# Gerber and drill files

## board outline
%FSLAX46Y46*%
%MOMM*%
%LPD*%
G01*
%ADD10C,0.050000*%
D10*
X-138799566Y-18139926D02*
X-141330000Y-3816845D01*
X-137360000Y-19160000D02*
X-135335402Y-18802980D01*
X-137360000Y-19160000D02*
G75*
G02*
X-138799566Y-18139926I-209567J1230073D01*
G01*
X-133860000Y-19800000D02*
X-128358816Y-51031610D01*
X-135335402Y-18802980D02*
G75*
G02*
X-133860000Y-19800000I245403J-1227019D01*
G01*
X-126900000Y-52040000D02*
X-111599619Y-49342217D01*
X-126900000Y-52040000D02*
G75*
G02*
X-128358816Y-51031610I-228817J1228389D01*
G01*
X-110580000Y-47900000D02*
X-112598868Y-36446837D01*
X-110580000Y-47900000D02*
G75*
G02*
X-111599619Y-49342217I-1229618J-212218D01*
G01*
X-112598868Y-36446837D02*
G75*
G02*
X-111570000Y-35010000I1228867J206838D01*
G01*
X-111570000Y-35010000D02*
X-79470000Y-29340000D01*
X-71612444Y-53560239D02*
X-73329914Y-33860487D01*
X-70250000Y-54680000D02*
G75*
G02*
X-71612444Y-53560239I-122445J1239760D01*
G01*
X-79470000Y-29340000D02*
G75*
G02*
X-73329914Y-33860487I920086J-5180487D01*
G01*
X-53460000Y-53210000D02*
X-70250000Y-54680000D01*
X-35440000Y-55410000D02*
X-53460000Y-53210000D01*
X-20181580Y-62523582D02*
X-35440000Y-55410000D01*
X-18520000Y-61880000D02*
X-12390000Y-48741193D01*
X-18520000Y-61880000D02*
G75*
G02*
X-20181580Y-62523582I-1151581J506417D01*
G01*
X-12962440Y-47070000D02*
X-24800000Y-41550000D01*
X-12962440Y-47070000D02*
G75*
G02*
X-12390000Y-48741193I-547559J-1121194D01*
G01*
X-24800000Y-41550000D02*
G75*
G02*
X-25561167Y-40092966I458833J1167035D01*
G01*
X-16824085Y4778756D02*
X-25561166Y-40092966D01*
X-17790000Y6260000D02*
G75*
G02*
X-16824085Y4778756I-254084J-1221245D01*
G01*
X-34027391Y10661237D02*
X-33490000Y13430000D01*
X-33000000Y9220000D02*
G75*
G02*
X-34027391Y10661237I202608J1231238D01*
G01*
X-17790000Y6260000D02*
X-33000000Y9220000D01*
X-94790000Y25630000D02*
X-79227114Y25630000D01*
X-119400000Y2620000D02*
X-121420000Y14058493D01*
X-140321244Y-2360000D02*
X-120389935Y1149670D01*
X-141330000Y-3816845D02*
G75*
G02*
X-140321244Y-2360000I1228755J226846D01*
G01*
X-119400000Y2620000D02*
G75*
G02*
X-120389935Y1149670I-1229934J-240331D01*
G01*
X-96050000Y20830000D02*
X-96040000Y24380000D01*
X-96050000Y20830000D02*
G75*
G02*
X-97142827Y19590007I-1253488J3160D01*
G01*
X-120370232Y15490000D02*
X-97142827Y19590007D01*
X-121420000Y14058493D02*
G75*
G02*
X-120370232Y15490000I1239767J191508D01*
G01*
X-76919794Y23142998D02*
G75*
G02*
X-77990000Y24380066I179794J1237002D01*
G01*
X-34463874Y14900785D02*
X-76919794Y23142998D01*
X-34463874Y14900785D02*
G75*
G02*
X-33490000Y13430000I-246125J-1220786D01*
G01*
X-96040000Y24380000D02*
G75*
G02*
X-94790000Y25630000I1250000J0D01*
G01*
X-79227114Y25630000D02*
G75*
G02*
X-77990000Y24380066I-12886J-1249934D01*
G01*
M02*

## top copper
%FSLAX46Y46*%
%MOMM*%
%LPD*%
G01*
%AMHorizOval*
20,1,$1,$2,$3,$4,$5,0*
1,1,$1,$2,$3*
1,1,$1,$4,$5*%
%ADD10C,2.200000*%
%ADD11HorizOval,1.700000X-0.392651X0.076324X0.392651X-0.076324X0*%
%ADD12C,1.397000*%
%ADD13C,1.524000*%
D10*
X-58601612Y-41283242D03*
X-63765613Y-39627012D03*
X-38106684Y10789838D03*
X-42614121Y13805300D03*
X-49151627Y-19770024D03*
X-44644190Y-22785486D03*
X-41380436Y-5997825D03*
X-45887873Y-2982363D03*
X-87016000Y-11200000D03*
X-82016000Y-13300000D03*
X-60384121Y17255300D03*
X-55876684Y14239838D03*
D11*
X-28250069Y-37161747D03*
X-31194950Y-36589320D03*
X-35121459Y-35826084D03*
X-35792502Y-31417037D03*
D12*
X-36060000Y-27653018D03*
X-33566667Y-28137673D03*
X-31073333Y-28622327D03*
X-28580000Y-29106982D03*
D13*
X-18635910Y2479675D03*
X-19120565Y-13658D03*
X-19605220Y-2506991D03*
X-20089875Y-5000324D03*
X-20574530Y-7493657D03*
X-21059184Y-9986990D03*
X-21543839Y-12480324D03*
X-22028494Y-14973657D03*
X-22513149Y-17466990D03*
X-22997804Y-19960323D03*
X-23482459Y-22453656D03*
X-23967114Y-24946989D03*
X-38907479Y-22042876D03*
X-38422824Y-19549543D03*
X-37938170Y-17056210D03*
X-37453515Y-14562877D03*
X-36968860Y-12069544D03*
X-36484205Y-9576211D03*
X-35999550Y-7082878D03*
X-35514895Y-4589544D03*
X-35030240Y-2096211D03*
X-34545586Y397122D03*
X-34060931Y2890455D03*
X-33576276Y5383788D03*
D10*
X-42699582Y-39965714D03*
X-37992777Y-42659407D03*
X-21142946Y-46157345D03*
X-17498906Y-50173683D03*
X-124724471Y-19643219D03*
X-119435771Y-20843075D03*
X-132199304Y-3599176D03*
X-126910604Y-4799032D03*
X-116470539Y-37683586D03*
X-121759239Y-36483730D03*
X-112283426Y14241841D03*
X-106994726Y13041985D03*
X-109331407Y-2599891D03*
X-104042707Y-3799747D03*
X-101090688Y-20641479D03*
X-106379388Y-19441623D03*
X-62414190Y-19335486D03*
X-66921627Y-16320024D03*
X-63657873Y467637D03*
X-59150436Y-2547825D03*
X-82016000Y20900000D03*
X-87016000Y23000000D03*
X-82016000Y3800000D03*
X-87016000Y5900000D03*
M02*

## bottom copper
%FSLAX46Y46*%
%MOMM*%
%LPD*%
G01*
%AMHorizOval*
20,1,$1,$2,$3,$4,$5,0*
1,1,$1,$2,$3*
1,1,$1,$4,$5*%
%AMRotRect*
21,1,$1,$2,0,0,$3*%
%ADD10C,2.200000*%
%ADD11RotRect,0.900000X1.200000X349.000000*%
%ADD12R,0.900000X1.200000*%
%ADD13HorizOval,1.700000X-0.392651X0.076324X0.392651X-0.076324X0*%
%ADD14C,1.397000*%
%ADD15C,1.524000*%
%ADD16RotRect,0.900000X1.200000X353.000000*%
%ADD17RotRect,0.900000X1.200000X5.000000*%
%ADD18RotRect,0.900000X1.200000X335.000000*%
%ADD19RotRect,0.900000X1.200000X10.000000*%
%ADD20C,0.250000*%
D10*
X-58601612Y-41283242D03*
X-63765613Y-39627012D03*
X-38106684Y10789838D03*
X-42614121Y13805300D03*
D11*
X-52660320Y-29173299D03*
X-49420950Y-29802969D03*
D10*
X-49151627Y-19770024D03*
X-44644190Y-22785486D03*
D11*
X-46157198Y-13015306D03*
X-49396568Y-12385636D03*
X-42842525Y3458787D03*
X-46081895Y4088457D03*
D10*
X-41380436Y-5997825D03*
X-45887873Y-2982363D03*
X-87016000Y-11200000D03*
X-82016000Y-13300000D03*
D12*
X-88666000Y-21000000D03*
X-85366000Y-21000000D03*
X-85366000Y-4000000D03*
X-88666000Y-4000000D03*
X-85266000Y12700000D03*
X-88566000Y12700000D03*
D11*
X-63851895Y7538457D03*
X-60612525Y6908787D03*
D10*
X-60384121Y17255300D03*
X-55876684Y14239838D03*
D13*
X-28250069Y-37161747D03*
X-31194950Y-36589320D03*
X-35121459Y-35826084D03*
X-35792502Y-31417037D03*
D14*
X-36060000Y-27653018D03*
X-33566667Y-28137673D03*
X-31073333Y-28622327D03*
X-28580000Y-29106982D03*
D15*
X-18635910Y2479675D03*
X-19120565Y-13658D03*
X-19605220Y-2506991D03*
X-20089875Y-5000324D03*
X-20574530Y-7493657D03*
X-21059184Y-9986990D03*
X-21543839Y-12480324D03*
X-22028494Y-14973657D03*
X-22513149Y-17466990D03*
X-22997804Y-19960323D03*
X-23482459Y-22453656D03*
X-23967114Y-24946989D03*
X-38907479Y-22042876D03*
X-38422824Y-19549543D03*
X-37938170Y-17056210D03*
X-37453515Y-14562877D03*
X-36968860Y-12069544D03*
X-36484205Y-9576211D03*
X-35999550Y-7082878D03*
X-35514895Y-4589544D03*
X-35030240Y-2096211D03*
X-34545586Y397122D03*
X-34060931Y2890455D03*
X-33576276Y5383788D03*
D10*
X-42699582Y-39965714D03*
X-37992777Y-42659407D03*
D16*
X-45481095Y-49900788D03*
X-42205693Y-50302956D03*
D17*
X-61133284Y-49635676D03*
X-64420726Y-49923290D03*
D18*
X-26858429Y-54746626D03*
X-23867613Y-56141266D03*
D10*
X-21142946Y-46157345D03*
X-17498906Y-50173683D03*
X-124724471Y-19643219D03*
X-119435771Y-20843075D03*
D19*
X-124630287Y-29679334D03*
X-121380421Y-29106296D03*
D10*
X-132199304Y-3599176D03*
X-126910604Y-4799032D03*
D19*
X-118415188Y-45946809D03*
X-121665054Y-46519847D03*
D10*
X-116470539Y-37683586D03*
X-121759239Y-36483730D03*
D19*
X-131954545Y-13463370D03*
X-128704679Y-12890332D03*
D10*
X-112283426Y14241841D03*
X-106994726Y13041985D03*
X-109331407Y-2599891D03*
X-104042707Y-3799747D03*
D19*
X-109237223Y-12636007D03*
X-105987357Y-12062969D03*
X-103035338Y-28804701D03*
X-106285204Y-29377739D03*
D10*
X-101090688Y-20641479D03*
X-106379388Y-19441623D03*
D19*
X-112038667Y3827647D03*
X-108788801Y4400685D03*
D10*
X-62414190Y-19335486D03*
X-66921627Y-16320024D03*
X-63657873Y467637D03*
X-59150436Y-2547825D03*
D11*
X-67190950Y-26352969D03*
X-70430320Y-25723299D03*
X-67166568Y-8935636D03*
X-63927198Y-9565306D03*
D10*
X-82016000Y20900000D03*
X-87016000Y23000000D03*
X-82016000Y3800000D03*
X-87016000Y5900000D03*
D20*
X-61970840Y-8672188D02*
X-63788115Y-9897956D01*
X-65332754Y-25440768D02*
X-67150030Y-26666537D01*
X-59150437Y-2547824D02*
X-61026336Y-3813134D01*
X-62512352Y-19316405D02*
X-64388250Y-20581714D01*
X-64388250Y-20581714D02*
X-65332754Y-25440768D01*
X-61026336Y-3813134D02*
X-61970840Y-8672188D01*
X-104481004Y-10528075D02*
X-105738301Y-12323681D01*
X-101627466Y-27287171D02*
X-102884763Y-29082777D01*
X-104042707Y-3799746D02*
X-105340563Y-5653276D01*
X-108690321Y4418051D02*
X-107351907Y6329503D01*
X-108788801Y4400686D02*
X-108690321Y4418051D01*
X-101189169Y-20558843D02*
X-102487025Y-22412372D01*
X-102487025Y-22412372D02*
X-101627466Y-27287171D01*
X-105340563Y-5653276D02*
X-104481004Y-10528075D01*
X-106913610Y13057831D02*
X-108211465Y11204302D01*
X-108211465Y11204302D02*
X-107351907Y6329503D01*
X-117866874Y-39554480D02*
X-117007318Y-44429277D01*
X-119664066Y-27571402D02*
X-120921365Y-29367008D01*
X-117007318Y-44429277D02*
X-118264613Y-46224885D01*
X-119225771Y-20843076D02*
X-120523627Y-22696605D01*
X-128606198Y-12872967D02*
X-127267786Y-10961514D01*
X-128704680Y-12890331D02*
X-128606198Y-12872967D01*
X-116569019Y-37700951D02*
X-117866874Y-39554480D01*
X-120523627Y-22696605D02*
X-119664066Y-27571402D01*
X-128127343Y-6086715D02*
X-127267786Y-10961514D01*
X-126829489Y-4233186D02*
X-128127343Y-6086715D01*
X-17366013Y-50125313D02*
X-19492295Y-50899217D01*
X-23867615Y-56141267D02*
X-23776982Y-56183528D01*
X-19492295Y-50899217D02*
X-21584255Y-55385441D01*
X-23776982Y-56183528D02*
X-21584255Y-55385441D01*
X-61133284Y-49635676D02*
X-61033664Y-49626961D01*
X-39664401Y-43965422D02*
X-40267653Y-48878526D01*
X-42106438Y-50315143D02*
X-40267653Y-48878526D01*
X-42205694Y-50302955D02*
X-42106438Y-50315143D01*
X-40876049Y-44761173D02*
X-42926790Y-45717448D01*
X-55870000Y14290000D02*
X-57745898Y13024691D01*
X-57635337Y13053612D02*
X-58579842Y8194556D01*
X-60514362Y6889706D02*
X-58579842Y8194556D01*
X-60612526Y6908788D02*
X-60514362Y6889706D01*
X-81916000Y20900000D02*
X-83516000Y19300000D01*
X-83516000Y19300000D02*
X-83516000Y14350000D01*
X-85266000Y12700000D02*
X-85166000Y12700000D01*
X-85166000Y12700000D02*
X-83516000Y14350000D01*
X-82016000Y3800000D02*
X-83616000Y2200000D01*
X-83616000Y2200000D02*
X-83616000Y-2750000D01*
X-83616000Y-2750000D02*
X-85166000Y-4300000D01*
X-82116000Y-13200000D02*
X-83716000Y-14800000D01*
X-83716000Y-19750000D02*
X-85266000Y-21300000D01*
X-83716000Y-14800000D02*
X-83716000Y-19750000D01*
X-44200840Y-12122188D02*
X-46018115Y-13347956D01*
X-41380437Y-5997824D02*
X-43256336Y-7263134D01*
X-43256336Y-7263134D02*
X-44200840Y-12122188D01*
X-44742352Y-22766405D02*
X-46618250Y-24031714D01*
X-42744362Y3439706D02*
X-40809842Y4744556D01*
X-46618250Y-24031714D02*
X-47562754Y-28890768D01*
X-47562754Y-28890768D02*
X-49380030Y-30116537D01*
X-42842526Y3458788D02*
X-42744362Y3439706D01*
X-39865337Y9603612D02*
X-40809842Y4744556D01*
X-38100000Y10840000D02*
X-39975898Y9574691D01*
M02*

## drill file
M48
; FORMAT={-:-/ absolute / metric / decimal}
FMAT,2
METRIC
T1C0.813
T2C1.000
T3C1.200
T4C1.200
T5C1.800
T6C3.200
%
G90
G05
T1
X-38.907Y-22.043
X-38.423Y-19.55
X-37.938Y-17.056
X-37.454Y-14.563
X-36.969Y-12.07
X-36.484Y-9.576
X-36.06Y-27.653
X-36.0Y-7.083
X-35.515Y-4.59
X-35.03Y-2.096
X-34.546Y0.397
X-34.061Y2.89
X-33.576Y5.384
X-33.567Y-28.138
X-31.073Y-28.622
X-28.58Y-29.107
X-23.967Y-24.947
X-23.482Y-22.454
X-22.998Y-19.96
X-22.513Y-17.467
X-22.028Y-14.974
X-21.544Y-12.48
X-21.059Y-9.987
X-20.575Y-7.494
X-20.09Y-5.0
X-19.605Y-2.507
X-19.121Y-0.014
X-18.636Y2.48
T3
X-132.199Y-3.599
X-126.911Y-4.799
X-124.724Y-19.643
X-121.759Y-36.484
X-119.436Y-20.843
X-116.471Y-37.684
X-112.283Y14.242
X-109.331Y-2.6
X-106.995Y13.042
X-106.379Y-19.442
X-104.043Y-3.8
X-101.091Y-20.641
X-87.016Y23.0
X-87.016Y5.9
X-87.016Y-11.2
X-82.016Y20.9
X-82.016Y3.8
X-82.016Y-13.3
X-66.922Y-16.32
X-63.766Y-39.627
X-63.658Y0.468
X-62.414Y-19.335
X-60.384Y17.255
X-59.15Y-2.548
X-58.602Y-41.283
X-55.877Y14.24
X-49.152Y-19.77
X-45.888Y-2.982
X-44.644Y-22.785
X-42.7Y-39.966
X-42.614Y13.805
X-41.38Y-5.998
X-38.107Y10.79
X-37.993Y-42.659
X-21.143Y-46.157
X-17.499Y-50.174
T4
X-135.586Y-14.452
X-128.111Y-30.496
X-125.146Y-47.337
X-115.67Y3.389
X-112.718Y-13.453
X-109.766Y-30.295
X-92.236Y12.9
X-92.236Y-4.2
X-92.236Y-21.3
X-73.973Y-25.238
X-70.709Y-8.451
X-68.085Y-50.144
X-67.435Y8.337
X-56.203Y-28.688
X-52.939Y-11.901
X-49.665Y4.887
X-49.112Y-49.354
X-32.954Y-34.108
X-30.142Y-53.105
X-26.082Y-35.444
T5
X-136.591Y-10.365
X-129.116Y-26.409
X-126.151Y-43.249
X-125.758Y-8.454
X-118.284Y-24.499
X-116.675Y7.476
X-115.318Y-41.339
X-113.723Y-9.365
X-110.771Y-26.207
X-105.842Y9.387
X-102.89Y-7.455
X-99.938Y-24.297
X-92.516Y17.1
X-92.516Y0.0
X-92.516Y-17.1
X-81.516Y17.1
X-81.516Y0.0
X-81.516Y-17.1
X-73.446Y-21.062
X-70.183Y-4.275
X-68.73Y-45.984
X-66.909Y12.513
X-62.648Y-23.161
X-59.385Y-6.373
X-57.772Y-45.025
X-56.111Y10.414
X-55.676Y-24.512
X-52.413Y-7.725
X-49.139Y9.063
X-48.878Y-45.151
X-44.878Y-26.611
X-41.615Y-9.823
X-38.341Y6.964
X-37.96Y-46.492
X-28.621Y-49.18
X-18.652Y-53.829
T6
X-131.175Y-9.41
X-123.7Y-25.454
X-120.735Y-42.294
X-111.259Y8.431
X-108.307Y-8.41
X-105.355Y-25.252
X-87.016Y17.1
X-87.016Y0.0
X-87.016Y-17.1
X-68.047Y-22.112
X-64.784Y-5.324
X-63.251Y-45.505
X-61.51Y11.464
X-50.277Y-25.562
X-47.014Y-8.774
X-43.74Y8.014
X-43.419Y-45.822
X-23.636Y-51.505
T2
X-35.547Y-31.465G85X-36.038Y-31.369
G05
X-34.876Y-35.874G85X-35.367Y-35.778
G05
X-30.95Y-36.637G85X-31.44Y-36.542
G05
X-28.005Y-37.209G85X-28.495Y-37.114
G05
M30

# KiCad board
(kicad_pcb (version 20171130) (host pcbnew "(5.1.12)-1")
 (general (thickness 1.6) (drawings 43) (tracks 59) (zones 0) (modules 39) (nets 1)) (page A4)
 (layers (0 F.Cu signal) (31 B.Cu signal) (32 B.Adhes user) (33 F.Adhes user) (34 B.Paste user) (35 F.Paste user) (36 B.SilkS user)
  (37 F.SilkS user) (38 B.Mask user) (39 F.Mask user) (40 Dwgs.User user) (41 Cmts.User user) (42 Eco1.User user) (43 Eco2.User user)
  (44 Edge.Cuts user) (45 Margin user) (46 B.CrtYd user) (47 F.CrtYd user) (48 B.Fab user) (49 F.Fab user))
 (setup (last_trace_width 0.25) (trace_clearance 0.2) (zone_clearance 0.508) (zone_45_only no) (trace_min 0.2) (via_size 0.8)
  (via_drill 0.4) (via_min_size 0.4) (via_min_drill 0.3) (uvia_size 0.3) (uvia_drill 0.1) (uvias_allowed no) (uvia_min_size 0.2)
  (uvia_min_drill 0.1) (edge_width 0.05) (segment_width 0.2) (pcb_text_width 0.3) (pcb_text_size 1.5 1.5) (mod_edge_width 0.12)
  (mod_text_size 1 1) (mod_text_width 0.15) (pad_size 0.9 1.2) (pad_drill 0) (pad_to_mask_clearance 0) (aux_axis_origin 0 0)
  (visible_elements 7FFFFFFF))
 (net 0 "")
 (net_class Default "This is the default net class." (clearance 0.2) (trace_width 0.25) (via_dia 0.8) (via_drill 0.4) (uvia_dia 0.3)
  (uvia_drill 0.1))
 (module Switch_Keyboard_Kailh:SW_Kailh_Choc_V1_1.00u (layer F.Cu) (at -63.251394 45.504561 5)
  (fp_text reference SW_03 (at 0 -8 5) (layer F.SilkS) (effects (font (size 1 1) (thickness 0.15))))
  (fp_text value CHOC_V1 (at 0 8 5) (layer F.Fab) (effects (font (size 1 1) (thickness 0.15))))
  (pad "" np_thru_hole circle (at -5.22 4.2 5) (size 1.2 1.2) (drill 1.2) (layers *.Cu *.Mask))
  (pad "" np_thru_hole circle (at 5.5 0 5) (size 1.8 1.8) (drill 1.8) (layers *.Cu *.Mask))
  (pad "" np_thru_hole circle (at -5.5 0 5) (size 1.8 1.8) (drill 1.8) (layers *.Cu *.Mask))
  (pad "" np_thru_hole circle (at 0 0 5) (size 3.2 3.2) (drill 3.2) (layers *.Cu *.Mask))
  (pad 2 thru_hole circle (at 5 -3.8 5) (size 2.2 2.2) (drill 1.2) (layers *.Cu B.Mask))
  (pad 1 thru_hole circle (at 0 -5.9 5) (size 2.2 2.2) (drill 1.2) (layers *.Cu B.Mask)))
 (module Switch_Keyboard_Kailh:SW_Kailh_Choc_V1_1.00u (layer F.Cu) (at -43.739894 -8.0137 349)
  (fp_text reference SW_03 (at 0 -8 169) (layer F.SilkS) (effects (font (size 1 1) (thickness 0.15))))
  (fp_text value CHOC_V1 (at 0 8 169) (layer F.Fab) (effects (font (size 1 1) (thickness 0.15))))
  (pad "" np_thru_hole circle (at -5.22 4.2 349) (size 1.2 1.2) (drill 1.2) (layers *.Cu *.Mask))
  (pad "" np_thru_hole circle (at 5.5 0 349) (size 1.8 1.8) (drill 1.8) (layers *.Cu *.Mask))
  (pad "" np_thru_hole circle (at -5.5 0 349) (size 1.8 1.8) (drill 1.8) (layers *.Cu *.Mask))
  (pad "" np_thru_hole circle (at 0 0 349) (size 3.2 3.2) (drill 3.2) (layers *.Cu *.Mask))
  (pad 2 thru_hole circle (at 5 -3.8 349) (size 2.2 2.2) (drill 1.2) (layers *.Cu B.Mask))
  (pad 1 thru_hole circle (at 0 -5.9 349) (size 2.2 2.2) (drill 1.2) (layers *.Cu B.Mask)))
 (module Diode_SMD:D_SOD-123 (layer B.Cu) (at -51.040635 29.488134 349)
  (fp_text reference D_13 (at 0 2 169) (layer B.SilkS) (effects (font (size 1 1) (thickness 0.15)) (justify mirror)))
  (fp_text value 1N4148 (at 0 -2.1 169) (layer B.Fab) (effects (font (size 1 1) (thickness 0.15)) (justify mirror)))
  (pad 1 smd rect (at -1.65 0 349) (size 0.9 1.2) (layers B.Cu B.Paste B.Mask))
  (pad 2 smd rect (at 1.65 0 349) (size 0.9 1.2) (layers B.Cu B.Paste B.Mask)))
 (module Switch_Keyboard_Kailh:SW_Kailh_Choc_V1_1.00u (layer F.Cu) (at -50.2774 25.561624 349)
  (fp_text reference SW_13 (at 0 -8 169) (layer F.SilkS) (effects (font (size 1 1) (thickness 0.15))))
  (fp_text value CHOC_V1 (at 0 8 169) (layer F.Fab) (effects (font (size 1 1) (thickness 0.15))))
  (pad 1 thru_hole circle (at 0 -5.9 349) (size 2.2 2.2) (drill 1.2) (layers *.Cu B.Mask))
  (pad 2 thru_hole circle (at 5 -3.8 349) (size 2.2 2.2) (drill 1.2) (layers *.Cu B.Mask))
  (pad "" np_thru_hole circle (at 0 0 349) (size 3.2 3.2) (drill 3.2) (layers *.Cu *.Mask))
  (pad "" np_thru_hole circle (at -5.5 0 349) (size 1.8 1.8) (drill 1.8) (layers *.Cu *.Mask))
  (pad "" np_thru_hole circle (at 5.5 0 349) (size 1.8 1.8) (drill 1.8) (layers *.Cu *.Mask))
  (pad "" np_thru_hole circle (at -5.22 4.2 349) (size 1.2 1.2) (drill 1.2) (layers *.Cu *.Mask)))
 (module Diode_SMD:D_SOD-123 (layer B.Cu) (at -47.776883 12.700471 349)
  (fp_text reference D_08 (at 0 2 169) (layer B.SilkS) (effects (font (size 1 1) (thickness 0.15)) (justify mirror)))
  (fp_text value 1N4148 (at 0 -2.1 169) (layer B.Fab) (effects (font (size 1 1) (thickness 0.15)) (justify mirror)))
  (pad 2 smd rect (at 1.65 0 349) (size 0.9 1.2) (layers B.Cu B.Paste B.Mask))
  (pad 1 smd rect (at -1.65 0 349) (size 0.9 1.2) (layers B.Cu B.Paste B.Mask)))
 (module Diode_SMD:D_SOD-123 (layer B.Cu) (at -44.46221 -3.773622 349)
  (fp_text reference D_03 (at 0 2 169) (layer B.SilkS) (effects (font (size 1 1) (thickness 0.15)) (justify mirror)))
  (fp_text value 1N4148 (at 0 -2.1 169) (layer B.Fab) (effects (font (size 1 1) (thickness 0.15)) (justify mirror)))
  (pad 2 smd rect (at 1.65 0 349) (size 0.9 1.2) (layers B.Cu B.Paste B.Mask))
  (pad 1 smd rect (at -1.65 0 349) (size 0.9 1.2) (layers B.Cu B.Paste B.Mask)))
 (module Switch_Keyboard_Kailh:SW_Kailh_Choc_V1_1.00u (layer F.Cu) (at -47.013646 8.773963 349)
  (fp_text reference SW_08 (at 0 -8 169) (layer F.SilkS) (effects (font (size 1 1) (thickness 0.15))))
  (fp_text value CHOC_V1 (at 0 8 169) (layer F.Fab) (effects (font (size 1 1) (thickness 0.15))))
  (pad "" np_thru_hole circle (at -5.22 4.2 349) (size 1.2 1.2) (drill 1.2) (layers *.Cu *.Mask))
  (pad "" np_thru_hole circle (at 5.5 0 349) (size 1.8 1.8) (drill 1.8) (layers *.Cu *.Mask))
  (pad "" np_thru_hole circle (at -5.5 0 349) (size 1.8 1.8) (drill 1.8) (layers *.Cu *.Mask))
  (pad "" np_thru_hole circle (at 0 0 349) (size 3.2 3.2) (drill 3.2) (layers *.Cu *.Mask))
  (pad 2 thru_hole circle (at 5 -3.8 349) (size 2.2 2.2) (drill 1.2) (layers *.Cu B.Mask))
  (pad 1 thru_hole circle (at 0 -5.9 349) (size 2.2 2.2) (drill 1.2) (layers *.Cu B.Mask)))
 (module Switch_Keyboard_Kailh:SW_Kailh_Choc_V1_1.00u (layer F.Cu) (at -87.016 17.1)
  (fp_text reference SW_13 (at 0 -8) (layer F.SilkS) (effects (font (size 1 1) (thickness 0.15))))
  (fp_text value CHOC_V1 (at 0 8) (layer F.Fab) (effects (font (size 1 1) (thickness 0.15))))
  (pad 1 thru_hole circle (at 0 -5.9) (size 2.2 2.2) (drill 1.2) (layers *.Cu B.Mask))
  (pad 2 thru_hole circle (at 5 -3.8) (size 2.2 2.2) (drill 1.2) (layers *.Cu B.Mask))
  (pad "" np_thru_hole circle (at 0 0) (size 3.2 3.2) (drill 3.2) (layers *.Cu *.Mask))
  (pad "" np_thru_hole circle (at -5.5 0) (size 1.8 1.8) (drill 1.8) (layers *.Cu *.Mask))
  (pad "" np_thru_hole circle (at 5.5 0) (size 1.8 1.8) (drill 1.8) (layers *.Cu *.Mask))
  (pad "" np_thru_hole circle (at -5.22 4.2) (size 1.2 1.2) (drill 1.2) (layers *.Cu *.Mask)))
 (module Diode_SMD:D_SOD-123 (layer B.Cu) (at -87.016 21)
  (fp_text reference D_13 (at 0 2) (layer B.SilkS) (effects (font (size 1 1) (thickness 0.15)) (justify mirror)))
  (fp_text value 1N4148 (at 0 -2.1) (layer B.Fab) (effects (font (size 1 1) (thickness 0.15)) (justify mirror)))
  (pad 1 smd rect (at -1.65 0) (size 0.9 1.2) (layers B.Cu B.Paste B.Mask))
  (pad 2 smd rect (at 1.65 0) (size 0.9 1.2) (layers B.Cu B.Paste B.Mask)))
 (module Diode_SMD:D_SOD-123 (layer B.Cu) (at -87.016 4)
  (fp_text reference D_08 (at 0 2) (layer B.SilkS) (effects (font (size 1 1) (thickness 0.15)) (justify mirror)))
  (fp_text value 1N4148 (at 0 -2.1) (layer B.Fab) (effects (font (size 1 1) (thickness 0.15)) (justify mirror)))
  (pad 2 smd rect (at 1.65 0) (size 0.9 1.2) (layers B.Cu B.Paste B.Mask))
  (pad 1 smd rect (at -1.65 0) (size 0.9 1.2) (layers B.Cu B.Paste B.Mask)))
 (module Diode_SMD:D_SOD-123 (layer B.Cu) (at -86.916 -12.7)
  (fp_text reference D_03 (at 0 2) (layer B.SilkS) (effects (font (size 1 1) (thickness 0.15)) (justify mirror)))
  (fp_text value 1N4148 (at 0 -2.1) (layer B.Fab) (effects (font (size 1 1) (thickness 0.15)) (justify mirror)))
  (pad 2 smd rect (at 1.65 0) (size 0.9 1.2) (layers B.Cu B.Paste B.Mask))
  (pad 1 smd rect (at -1.65 0) (size 0.9 1.2) (layers B.Cu B.Paste B.Mask)))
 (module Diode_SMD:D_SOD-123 (layer B.Cu) (at -62.23221 -7.223622 349)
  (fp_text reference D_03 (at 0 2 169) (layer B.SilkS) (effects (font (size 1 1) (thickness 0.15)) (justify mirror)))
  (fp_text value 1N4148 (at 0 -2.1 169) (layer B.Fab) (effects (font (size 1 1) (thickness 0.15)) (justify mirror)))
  (pad 1 smd rect (at -1.65 0 349) (size 0.9 1.2) (layers B.Cu B.Paste B.Mask))
  (pad 2 smd rect (at 1.65 0 349) (size 0.9 1.2) (layers B.Cu B.Paste B.Mask)))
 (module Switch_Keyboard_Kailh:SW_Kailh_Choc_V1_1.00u (layer F.Cu) (at -61.509894 -11.4637 349)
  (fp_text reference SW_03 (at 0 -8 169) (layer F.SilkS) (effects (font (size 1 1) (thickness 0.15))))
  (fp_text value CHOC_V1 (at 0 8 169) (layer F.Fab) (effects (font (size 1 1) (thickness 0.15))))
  (pad 1 thru_hole circle (at 0 -5.9 349) (size 2.2 2.2) (drill 1.2) (layers *.Cu B.Mask))
  (pad 2 thru_hole circle (at 5 -3.8 349) (size 2.2 2.2) (drill 1.2) (layers *.Cu B.Mask))
  (pad "" np_thru_hole circle (at 0 0 349) (size 3.2 3.2) (drill 3.2) (layers *.Cu *.Mask))
  (pad "" np_thru_hole circle (at -5.5 0 349) (size 1.8 1.8) (drill 1.8) (layers *.Cu *.Mask))
  (pad "" np_thru_hole circle (at 5.5 0 349) (size 1.8 1.8) (drill 1.8) (layers *.Cu *.Mask))
  (pad "" np_thru_hole circle (at -5.22 4.2 349) (size 1.2 1.2) (drill 1.2) (layers *.Cu *.Mask)))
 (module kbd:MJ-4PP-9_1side (layer F.Cu) (at -24.61 35.73 259)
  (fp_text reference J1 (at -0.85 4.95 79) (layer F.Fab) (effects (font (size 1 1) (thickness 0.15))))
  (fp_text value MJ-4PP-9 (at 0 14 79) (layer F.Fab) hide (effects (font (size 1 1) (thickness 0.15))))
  (pad "" np_thru_hole circle (at 0 1.5 259) (size 1.2 1.2) (drill 1.2) (layers *.Cu *.Mask))
  (pad "" np_thru_hole circle (at 0 8.5 259) (size 1.2 1.2) (drill 1.2) (layers *.Cu *.Mask))
  (pad B thru_hole oval (at 2.1 3.3 259) (size 1.7 2.5) (drill oval 1 1.5) (layers *.Cu B.Mask))
  (pad C thru_hole oval (at 2.1 6.3 259) (size 1.7 2.5) (drill oval 1 1.5) (layers *.Cu B.Mask))
  (pad D thru_hole oval (at 2.1 10.3 259) (size 1.7 2.5) (drill oval 1 1.5) (layers *.Cu B.Mask) (clearance 0.15))
  (pad A thru_hole oval (at -2.1 11.8 259) (size 1.7 2.5) (drill oval 1 1.5) (layers *.Cu B.Mask) (clearance 0.15)))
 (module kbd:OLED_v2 (layer F.Cu) (at -32.32 28.38 349)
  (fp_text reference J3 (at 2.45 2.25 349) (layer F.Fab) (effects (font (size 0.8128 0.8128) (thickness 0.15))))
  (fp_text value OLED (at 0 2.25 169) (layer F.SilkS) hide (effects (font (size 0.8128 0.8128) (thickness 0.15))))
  (pad 1 thru_hole circle (at -3.81 0 349) (size 1.397 1.397) (drill 0.8128) (layers *.Cu F.SilkS B.Mask))
  (pad 2 thru_hole circle (at -1.27 0 349) (size 1.397 1.397) (drill 0.8128) (layers *.Cu F.SilkS B.Mask))
  (pad 3 thru_hole circle (at 1.27 0 349) (size 1.397 1.397) (drill 0.8128) (layers *.Cu F.SilkS B.Mask))
  (pad 4 thru_hole circle (at 3.81 0 349) (size 1.397 1.397) (drill 0.8128) (layers *.Cu F.SilkS B.Mask)))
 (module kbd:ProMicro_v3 (layer F.Cu) (at -28.87 10.28 349)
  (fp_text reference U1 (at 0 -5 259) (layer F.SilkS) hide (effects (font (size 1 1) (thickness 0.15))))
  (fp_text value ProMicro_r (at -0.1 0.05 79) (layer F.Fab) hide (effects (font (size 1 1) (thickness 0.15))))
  (pad 1 thru_hole circle (at 7.6114 -14.478 349) (size 1.524 1.524) (drill 0.8128) (layers *.Cu B.Mask))
  (pad 2 thru_hole circle (at 7.6114 -11.938 349) (size 1.524 1.524) (drill 0.8128) (layers *.Cu B.Mask))
  (pad 3 thru_hole circle (at 7.6114 -9.398 349) (size 1.524 1.524) (drill 0.8128) (layers *.Cu B.Mask))
  (pad 4 thru_hole circle (at 7.6114 -6.858 349) (size 1.524 1.524) (drill 0.8128) (layers *.Cu B.Mask))
  (pad 5 thru_hole circle (at 7.6114 -4.318 349) (size 1.524 1.524) (drill 0.8128) (layers *.Cu B.Mask))
  (pad 6 thru_hole circle (at 7.6114 -1.778 349) (size 1.524 1.524) (drill 0.8128) (layers *.Cu B.Mask))
  (pad 7 thru_hole circle (at 7.6114 0.762 349) (size 1.524 1.524) (drill 0.8128) (layers *.Cu B.Mask))
  (pad 8 thru_hole circle (at 7.6114 3.302 349) (size 1.524 1.524) (drill 0.8128) (layers *.Cu B.Mask))
  (pad 9 thru_hole circle (at 7.6114 5.842 349) (size 1.524 1.524) (drill 0.8128) (layers *.Cu B.Mask))
  (pad 10 thru_hole circle (at 7.6114 8.382 349) (size 1.524 1.524) (drill 0.8128) (layers *.Cu B.Mask))
  (pad 11 thru_hole circle (at 7.6114 10.922 349) (size 1.524 1.524) (drill 0.8128) (layers *.Cu B.Mask))
  (pad 12 thru_hole circle (at 7.6114 13.462 349) (size 1.524 1.524) (drill 0.8128) (layers *.Cu B.Mask))
  (pad 13 thru_hole circle (at -7.6086 13.462 349) (size 1.524 1.524) (drill 0.8128) (layers *.Cu B.Mask))
  (pad 14 thru_hole circle (at -7.6086 10.922 349) (size 1.524 1.524) (drill 0.8128) (layers *.Cu B.Mask))
  (pad 15 thru_hole circle (at -7.6086 8.382 349) (size 1.524 1.524) (drill 0.8128) (layers *.Cu B.Mask))
  (pad 16 thru_hole circle (at -7.6086 5.842 349) (size 1.524 1.524) (drill 0.8128) (layers *.Cu B.Mask))
  (pad 17 thru_hole circle (at -7.6086 3.302 349) (size 1.524 1.524) (drill 0.8128) (layers *.Cu B.Mask))
  (pad 18 thru_hole circle (at -7.6086 0.762 349) (size 1.524 1.524) (drill 0.8128) (layers *.Cu B.Mask))
  (pad 19 thru_hole circle (at -7.6086 -1.778 349) (size 1.524 1.524) (drill 0.8128) (layers *.Cu B.Mask))
  (pad 20 thru_hole circle (at -7.6086 -4.318 349) (size 1.524 1.524) (drill 0.8128) (layers *.Cu B.Mask))
  (pad 21 thru_hole circle (at -7.6086 -6.858 349) (size 1.524 1.524) (drill 0.8128) (layers *.Cu B.Mask))
  (pad 22 thru_hole circle (at -7.6086 -9.398 349) (size 1.524 1.524) (drill 0.8128) (layers *.Cu B.Mask))
  (pad 23 thru_hole circle (at -7.6086 -11.938 349) (size 1.524 1.524) (drill 0.8128) (layers *.Cu B.Mask))
  (pad 24 thru_hole circle (at -7.6086 -14.478 349) (size 1.524 1.524) (drill 0.8128) (layers *.Cu B.Mask)))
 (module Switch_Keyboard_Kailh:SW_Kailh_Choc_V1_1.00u (layer F.Cu) (at -43.418611 45.821736 353)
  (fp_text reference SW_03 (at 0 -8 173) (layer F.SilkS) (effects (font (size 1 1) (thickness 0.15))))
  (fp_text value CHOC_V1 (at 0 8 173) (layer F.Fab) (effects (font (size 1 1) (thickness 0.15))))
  (pad 1 thru_hole circle (at 0 -5.9 353) (size 2.2 2.2) (drill 1.2) (layers *.Cu B.Mask))
  (pad 2 thru_hole circle (at 5 -3.8 353) (size 2.2 2.2) (drill 1.2) (layers *.Cu B.Mask))
  (pad "" np_thru_hole circle (at 0 0 353) (size 3.2 3.2) (drill 3.2) (layers *.Cu *.Mask))
  (pad "" np_thru_hole circle (at -5.5 0 353) (size 1.8 1.8) (drill 1.8) (layers *.Cu *.Mask))
  (pad "" np_thru_hole circle (at 5.5 0 353) (size 1.8 1.8) (drill 1.8) (layers *.Cu *.Mask))
  (pad "" np_thru_hole circle (at -5.22 4.2 353) (size 1.2 1.2) (drill 1.2) (layers *.Cu *.Mask)))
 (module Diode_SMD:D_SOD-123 (layer B.Cu) (at -43.843394 50.101872 353)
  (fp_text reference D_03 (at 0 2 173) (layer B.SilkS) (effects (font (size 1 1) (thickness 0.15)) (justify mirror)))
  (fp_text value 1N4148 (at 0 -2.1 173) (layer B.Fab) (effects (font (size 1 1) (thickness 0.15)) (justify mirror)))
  (pad 1 smd rect (at -1.65 0 353) (size 0.9 1.2) (layers B.Cu B.Paste B.Mask))
  (pad 2 smd rect (at 1.65 0 353) (size 0.9 1.2) (layers B.Cu B.Paste B.Mask)))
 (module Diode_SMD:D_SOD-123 (layer B.Cu) (at -62.777005 49.779483 5)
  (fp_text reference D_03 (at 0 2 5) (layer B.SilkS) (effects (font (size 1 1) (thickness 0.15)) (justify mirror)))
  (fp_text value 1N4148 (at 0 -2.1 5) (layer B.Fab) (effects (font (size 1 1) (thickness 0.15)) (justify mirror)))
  (pad 2 smd rect (at 1.65 0 5) (size 0.9 1.2) (layers B.Cu B.Paste B.Mask))
  (pad 1 smd rect (at -1.65 0 5) (size 0.9 1.2) (layers B.Cu B.Paste B.Mask)))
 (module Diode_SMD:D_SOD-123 (layer B.Cu) (at -25.363021 55.443946 335)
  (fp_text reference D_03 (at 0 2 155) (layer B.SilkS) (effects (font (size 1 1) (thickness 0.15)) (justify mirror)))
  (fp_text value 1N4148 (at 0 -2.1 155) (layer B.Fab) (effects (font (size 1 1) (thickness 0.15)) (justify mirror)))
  (pad 1 smd rect (at -1.65 0 335) (size 0.9 1.2) (layers B.Cu B.Paste B.Mask))
  (pad 2 smd rect (at 1.65 0 335) (size 0.9 1.2) (layers B.Cu B.Paste B.Mask)))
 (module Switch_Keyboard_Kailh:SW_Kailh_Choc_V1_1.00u (layer F.Cu) (at -23.636394 51.504561 335)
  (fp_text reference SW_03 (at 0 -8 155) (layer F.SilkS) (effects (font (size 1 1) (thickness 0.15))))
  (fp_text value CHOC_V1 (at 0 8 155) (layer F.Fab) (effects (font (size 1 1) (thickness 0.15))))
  (pad 1 thru_hole circle (at 0 -5.9 335) (size 2.2 2.2) (drill 1.2) (layers *.Cu B.Mask))
  (pad 2 thru_hole circle (at 5 -3.8 335) (size 2.2 2.2) (drill 1.2) (layers *.Cu B.Mask))
  (pad "" np_thru_hole circle (at 0 0 335) (size 3.2 3.2) (drill 3.2) (layers *.Cu *.Mask))
  (pad "" np_thru_hole circle (at -5.5 0 335) (size 1.8 1.8) (drill 1.8) (layers *.Cu *.Mask))
  (pad "" np_thru_hole circle (at 5.5 0 335) (size 1.8 1.8) (drill 1.8) (layers *.Cu *.Mask))
  (pad "" np_thru_hole circle (at -5.22 4.2 335) (size 1.2 1.2) (drill 1.2) (layers *.Cu *.Mask)))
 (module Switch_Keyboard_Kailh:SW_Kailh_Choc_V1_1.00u (layer F.Cu) (at -123.699947 25.453585 10)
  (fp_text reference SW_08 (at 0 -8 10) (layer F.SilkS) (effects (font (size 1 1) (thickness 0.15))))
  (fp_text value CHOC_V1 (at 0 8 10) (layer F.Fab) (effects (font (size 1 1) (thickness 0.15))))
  (pad 1 thru_hole circle (at 0 -5.9 10) (size 2.2 2.2) (drill 1.2) (layers *.Cu B.Mask))
  (pad 2 thru_hole circle (at 5 -3.8 10) (size 2.2 2.2) (drill 1.2) (layers *.Cu B.Mask))
  (pad "" np_thru_hole circle (at 0 0 10) (size 3.2 3.2) (drill 3.2) (layers *.Cu *.Mask))
  (pad "" np_thru_hole circle (at -5.5 0 10) (size 1.8 1.8) (drill 1.8) (layers *.Cu *.Mask))
  (pad "" np_thru_hole circle (at 5.5 0 10) (size 1.8 1.8) (drill 1.8) (layers *.Cu *.Mask))
  (pad "" np_thru_hole circle (at -5.22 4.2 10) (size 1.2 1.2) (drill 1.2) (layers *.Cu *.Mask)))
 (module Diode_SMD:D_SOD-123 (layer B.Cu) (at -123.005354 29.392815 10)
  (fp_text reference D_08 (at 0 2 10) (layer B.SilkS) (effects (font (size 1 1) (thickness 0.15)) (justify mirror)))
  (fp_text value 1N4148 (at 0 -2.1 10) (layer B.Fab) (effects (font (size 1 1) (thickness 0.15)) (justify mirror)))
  (pad 1 smd rect (at -1.65 0 10) (size 0.9 1.2) (layers B.Cu B.Paste B.Mask))
  (pad 2 smd rect (at 1.65 0 10) (size 0.9 1.2) (layers B.Cu B.Paste B.Mask)))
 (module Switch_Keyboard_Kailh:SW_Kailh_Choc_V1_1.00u (layer F.Cu) (at -131.17478 9.409542 10)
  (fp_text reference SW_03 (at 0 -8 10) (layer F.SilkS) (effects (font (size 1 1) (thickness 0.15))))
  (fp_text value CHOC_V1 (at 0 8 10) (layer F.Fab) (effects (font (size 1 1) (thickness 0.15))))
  (pad 1 thru_hole circle (at 0 -5.9 10) (size 2.2 2.2) (drill 1.2) (layers *.Cu B.Mask))
  (pad 2 thru_hole circle (at 5 -3.8 10) (size 2.2 2.2) (drill 1.2) (layers *.Cu B.Mask))
  (pad "" np_thru_hole circle (at 0 0 10) (size 3.2 3.2) (drill 3.2) (layers *.Cu *.Mask))
  (pad "" np_thru_hole circle (at -5.5 0 10) (size 1.8 1.8) (drill 1.8) (layers *.Cu *.Mask))
  (pad "" np_thru_hole circle (at 5.5 0 10) (size 1.8 1.8) (drill 1.8) (layers *.Cu *.Mask))
  (pad "" np_thru_hole circle (at -5.22 4.2 10) (size 1.2 1.2) (drill 1.2) (layers *.Cu *.Mask)))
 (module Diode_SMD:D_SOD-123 (layer B.Cu) (at -120.040121 46.233328 10)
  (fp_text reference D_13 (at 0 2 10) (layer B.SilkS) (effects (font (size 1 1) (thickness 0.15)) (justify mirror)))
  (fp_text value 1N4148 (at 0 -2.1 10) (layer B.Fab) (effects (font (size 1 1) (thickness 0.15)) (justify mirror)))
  (pad 2 smd rect (at 1.65 0 10) (size 0.9 1.2) (layers B.Cu B.Paste B.Mask))
  (pad 1 smd rect (at -1.65 0 10) (size 0.9 1.2) (layers B.Cu B.Paste B.Mask)))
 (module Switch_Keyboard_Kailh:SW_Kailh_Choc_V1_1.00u (layer F.Cu) (at -120.734715 42.294096 10)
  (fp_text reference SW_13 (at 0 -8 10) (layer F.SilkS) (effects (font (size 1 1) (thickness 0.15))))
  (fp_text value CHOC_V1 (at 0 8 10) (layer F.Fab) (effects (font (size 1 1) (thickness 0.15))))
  (pad "" np_thru_hole circle (at -5.22 4.2 10) (size 1.2 1.2) (drill 1.2) (layers *.Cu *.Mask))
  (pad "" np_thru_hole circle (at 5.5 0 10) (size 1.8 1.8) (drill 1.8) (layers *.Cu *.Mask))
  (pad "" np_thru_hole circle (at -5.5 0 10) (size 1.8 1.8) (drill 1.8) (layers *.Cu *.Mask))
  (pad "" np_thru_hole circle (at 0 0 10) (size 3.2 3.2) (drill 3.2) (layers *.Cu *.Mask))
  (pad 2 thru_hole circle (at 5 -3.8 10) (size 2.2 2.2) (drill 1.2) (layers *.Cu B.Mask))
  (pad 1 thru_hole circle (at 0 -5.9 10) (size 2.2 2.2) (drill 1.2) (layers *.Cu B.Mask)))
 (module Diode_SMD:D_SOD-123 (layer B.Cu) (at -130.329612 13.176851 10)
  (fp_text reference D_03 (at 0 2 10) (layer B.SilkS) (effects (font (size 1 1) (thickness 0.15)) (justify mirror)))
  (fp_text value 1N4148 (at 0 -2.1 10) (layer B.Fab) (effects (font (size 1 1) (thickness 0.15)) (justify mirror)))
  (pad 1 smd rect (at -1.65 0 10) (size 0.9 1.2) (layers B.Cu B.Paste B.Mask))
  (pad 2 smd rect (at 1.65 0 10) (size 0.9 1.2) (layers B.Cu B.Paste B.Mask)))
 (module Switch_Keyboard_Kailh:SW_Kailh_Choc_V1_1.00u (layer F.Cu) (at -111.258902 -8.431475 10)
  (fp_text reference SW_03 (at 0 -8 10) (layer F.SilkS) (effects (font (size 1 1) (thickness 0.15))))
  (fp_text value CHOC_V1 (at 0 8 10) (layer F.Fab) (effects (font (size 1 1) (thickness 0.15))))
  (pad 1 thru_hole circle (at 0 -5.9 10) (size 2.2 2.2) (drill 1.2) (layers *.Cu B.Mask))
  (pad 2 thru_hole circle (at 5 -3.8 10) (size 2.2 2.2) (drill 1.2) (layers *.Cu B.Mask))
  (pad "" np_thru_hole circle (at 0 0 10) (size 3.2 3.2) (drill 3.2) (layers *.Cu *.Mask))
  (pad "" np_thru_hole circle (at -5.5 0 10) (size 1.8 1.8) (drill 1.8) (layers *.Cu *.Mask))
  (pad "" np_thru_hole circle (at 5.5 0 10) (size 1.8 1.8) (drill 1.8) (layers *.Cu *.Mask))
  (pad "" np_thru_hole circle (at -5.22 4.2 10) (size 1.2 1.2) (drill 1.2) (layers *.Cu *.Mask)))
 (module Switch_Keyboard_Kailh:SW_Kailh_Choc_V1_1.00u (layer F.Cu) (at -108.306883 8.410257 10)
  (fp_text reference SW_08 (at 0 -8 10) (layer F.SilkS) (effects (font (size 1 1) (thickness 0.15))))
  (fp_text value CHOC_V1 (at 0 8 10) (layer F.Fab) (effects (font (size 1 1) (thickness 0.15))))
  (pad 1 thru_hole circle (at 0 -5.9 10) (size 2.2 2.2) (drill 1.2) (layers *.Cu B.Mask))
  (pad 2 thru_hole circle (at 5 -3.8 10) (size 2.2 2.2) (drill 1.2) (layers *.Cu B.Mask))
  (pad "" np_thru_hole circle (at 0 0 10) (size 3.2 3.2) (drill 3.2) (layers *.Cu *.Mask))
  (pad "" np_thru_hole circle (at -5.5 0 10) (size 1.8 1.8) (drill 1.8) (layers *.Cu *.Mask))
  (pad "" np_thru_hole circle (at 5.5 0 10) (size 1.8 1.8) (drill 1.8) (layers *.Cu *.Mask))
  (pad "" np_thru_hole circle (at -5.22 4.2 10) (size 1.2 1.2) (drill 1.2) (layers *.Cu *.Mask)))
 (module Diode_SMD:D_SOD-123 (layer B.Cu) (at -107.61229 12.349488 10)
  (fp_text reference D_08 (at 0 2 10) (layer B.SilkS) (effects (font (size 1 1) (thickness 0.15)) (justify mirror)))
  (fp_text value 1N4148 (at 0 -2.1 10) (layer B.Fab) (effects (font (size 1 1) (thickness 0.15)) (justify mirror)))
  (pad 1 smd rect (at -1.65 0 10) (size 0.9 1.2) (layers B.Cu B.Paste B.Mask))
  (pad 2 smd rect (at 1.65 0 10) (size 0.9 1.2) (layers B.Cu B.Paste B.Mask)))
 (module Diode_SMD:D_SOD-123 (layer B.Cu) (at -104.660271 29.09122 10)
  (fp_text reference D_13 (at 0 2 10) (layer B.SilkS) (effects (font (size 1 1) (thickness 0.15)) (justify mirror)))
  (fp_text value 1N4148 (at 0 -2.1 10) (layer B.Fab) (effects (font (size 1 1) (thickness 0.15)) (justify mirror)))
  (pad 2 smd rect (at 1.65 0 10) (size 0.9 1.2) (layers B.Cu B.Paste B.Mask))
  (pad 1 smd rect (at -1.65 0 10) (size 0.9 1.2) (layers B.Cu B.Paste B.Mask)))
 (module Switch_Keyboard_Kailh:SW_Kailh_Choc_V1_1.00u (layer F.Cu) (at -105.354864 25.251989 10)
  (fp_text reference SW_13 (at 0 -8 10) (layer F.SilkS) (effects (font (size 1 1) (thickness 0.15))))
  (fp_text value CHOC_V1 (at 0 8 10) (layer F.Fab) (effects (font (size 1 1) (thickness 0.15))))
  (pad "" np_thru_hole circle (at -5.22 4.2 10) (size 1.2 1.2) (drill 1.2) (layers *.Cu *.Mask))
  (pad "" np_thru_hole circle (at 5.5 0 10) (size 1.8 1.8) (drill 1.8) (layers *.Cu *.Mask))
  (pad "" np_thru_hole circle (at -5.5 0 10) (size 1.8 1.8) (drill 1.8) (layers *.Cu *.Mask))
  (pad "" np_thru_hole circle (at 0 0 10) (size 3.2 3.2) (drill 3.2) (layers *.Cu *.Mask))
  (pad 2 thru_hole circle (at 5 -3.8 10) (size 2.2 2.2) (drill 1.2) (layers *.Cu B.Mask))
  (pad 1 thru_hole circle (at 0 -5.9 10) (size 2.2 2.2) (drill 1.2) (layers *.Cu B.Mask)))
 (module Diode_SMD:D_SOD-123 (layer B.Cu) (at -110.413734 -4.114166 10)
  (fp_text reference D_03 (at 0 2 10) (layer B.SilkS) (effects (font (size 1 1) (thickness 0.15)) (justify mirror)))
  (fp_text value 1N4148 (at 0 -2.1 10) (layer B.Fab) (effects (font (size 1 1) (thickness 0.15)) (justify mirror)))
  (pad 1 smd rect (at -1.65 0 10) (size 0.9 1.2) (layers B.Cu B.Paste B.Mask))
  (pad 2 smd rect (at 1.65 0 10) (size 0.9 1.2) (layers B.Cu B.Paste B.Mask)))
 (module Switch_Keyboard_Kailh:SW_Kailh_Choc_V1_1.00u (layer F.Cu) (at -68.0474 22.111624 349)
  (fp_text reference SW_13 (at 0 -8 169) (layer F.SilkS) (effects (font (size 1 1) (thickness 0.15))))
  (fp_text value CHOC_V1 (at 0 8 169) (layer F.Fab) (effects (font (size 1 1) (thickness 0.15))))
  (pad "" np_thru_hole circle (at -5.22 4.2 349) (size 1.2 1.2) (drill 1.2) (layers *.Cu *.Mask))
  (pad "" np_thru_hole circle (at 5.5 0 349) (size 1.8 1.8) (drill 1.8) (layers *.Cu *.Mask))
  (pad "" np_thru_hole circle (at -5.5 0 349) (size 1.8 1.8) (drill 1.8) (layers *.Cu *.Mask))
  (pad "" np_thru_hole circle (at 0 0 349) (size 3.2 3.2) (drill 3.2) (layers *.Cu *.Mask))
  (pad 2 thru_hole circle (at 5 -3.8 349) (size 2.2 2.2) (drill 1.2) (layers *.Cu B.Mask))
  (pad 1 thru_hole circle (at 0 -5.9 349) (size 2.2 2.2) (drill 1.2) (layers *.Cu B.Mask)))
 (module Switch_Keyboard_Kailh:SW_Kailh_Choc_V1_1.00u (layer F.Cu) (at -64.783646 5.323963 349)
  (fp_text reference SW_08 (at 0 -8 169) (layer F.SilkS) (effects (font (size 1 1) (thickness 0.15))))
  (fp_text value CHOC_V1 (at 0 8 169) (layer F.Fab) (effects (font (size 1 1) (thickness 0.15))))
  (pad 1 thru_hole circle (at 0 -5.9 349) (size 2.2 2.2) (drill 1.2) (layers *.Cu B.Mask))
  (pad 2 thru_hole circle (at 5 -3.8 349) (size 2.2 2.2) (drill 1.2) (layers *.Cu B.Mask))
  (pad "" np_thru_hole circle (at 0 0 349) (size 3.2 3.2) (drill 3.2) (layers *.Cu *.Mask))
  (pad "" np_thru_hole circle (at -5.5 0 349) (size 1.8 1.8) (drill 1.8) (layers *.Cu *.Mask))
  (pad "" np_thru_hole circle (at 5.5 0 349) (size 1.8 1.8) (drill 1.8) (layers *.Cu *.Mask))
  (pad "" np_thru_hole circle (at -5.22 4.2 349) (size 1.2 1.2) (drill 1.2) (layers *.Cu *.Mask)))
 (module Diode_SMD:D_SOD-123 (layer B.Cu) (at -68.810635 26.038134 349)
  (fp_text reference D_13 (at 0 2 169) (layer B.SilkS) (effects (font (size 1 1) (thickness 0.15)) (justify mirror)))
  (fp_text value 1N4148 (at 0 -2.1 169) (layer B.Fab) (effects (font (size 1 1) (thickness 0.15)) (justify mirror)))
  (pad 2 smd rect (at 1.65 0 349) (size 0.9 1.2) (layers B.Cu B.Paste B.Mask))
  (pad 1 smd rect (at -1.65 0 349) (size 0.9 1.2) (layers B.Cu B.Paste B.Mask)))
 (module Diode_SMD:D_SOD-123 (layer B.Cu) (at -65.546883 9.250471 349)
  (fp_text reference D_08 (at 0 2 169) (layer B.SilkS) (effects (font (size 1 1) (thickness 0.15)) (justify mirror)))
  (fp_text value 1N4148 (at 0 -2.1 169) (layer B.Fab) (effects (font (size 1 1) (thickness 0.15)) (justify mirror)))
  (pad 1 smd rect (at -1.65 0 349) (size 0.9 1.2) (layers B.Cu B.Paste B.Mask))
  (pad 2 smd rect (at 1.65 0 349) (size 0.9 1.2) (layers B.Cu B.Paste B.Mask)))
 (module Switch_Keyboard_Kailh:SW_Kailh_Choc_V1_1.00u (layer F.Cu) (at -87.016 -17.1)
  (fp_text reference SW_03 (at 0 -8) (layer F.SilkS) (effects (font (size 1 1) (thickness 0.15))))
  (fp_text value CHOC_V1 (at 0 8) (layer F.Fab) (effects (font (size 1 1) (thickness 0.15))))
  (pad "" np_thru_hole circle (at -5.22 4.2) (size 1.2 1.2) (drill 1.2) (layers *.Cu *.Mask))
  (pad "" np_thru_hole circle (at 5.5 0) (size 1.8 1.8) (drill 1.8) (layers *.Cu *.Mask))
  (pad "" np_thru_hole circle (at -5.5 0) (size 1.8 1.8) (drill 1.8) (layers *.Cu *.Mask))
  (pad "" np_thru_hole circle (at 0 0) (size 3.2 3.2) (drill 3.2) (layers *.Cu *.Mask))
  (pad 2 thru_hole circle (at 5 -3.8) (size 2.2 2.2) (drill 1.2) (layers *.Cu B.Mask))
  (pad 1 thru_hole circle (at 0 -5.9) (size 2.2 2.2) (drill 1.2) (layers *.Cu B.Mask)))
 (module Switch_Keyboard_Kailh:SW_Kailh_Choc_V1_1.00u (layer F.Cu) (at -87.016 0)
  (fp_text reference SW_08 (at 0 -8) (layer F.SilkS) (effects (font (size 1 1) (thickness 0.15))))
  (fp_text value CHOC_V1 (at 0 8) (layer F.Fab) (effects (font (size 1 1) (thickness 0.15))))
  (pad "" np_thru_hole circle (at -5.22 4.2) (size 1.2 1.2) (drill 1.2) (layers *.Cu *.Mask))
  (pad "" np_thru_hole circle (at 5.5 0) (size 1.8 1.8) (drill 1.8) (layers *.Cu *.Mask))
  (pad "" np_thru_hole circle (at -5.5 0) (size 1.8 1.8) (drill 1.8) (layers *.Cu *.Mask))
  (pad "" np_thru_hole circle (at 0 0) (size 3.2 3.2) (drill 3.2) (layers *.Cu *.Mask))
  (pad 2 thru_hole circle (at 5 -3.8) (size 2.2 2.2) (drill 1.2) (layers *.Cu B.Mask))
  (pad 1 thru_hole circle (at 0 -5.9) (size 2.2 2.2) (drill 1.2) (layers *.Cu B.Mask)))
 (gr_line (start -138.799566 18.139926) (end -141.33 3.816845) (layer Edge.Cuts) (width 0.05))
 (gr_line (start -137.36 19.16) (end -135.335402 18.80298) (layer Edge.Cuts) (width 0.05))
 (gr_arc (start -137.569567 17.929927) (end -138.799566 18.139926) (angle -89.9798821) (layer Edge.Cuts) (width 0.05))
 (gr_line (start -133.86 19.8) (end -128.358816 51.03161) (layer Edge.Cuts) (width 0.05))
 (gr_arc (start -135.089999 20.029999) (end -133.86 19.8) (angle -90.71840473) (layer Edge.Cuts) (width 0.05))
 (gr_line (start -126.9 52.04) (end -111.599619 49.342217) (layer Edge.Cuts) (width 0.05))
 (gr_arc (start -127.128817 50.811611) (end -128.358816 51.03161) (angle -90.41101636) (layer Edge.Cuts) (width 0.05))
 (gr_line (start -110.58 47.9) (end -112.598868 36.446837) (layer Edge.Cuts) (width 0.05))
 (gr_arc (start -111.809618 48.112218) (end -111.599619 49.342217) (angle -90.10335968) (layer Edge.Cuts) (width 0.05))
 (gr_arc (start -111.370001 36.239999) (end -111.57 35.01) (angle -90.31873058) (layer Edge.Cuts) (width 0.05))
 (gr_line (start -111.57 35.01) (end -79.47 29.34) (layer Edge.Cuts) (width 0.05))
 (gr_line (start -71.612444 53.560239) (end -73.329914 33.860487) (layer Edge.Cuts) (width 0.05))
 (gr_arc (start -70.372445 53.44024) (end -71.612444 53.560239) (angle -90.11300928) (layer Edge.Cuts) (width 0.05))
 (gr_arc (start -78.549914 34.520487) (end -73.329914 33.860487) (angle -92.86500996) (layer Edge.Cuts) (width 0.05))
 (gr_line (start -53.46 53.21) (end -70.25 54.68) (layer Edge.Cuts) (width 0.05))
 (gr_line (start -35.44 55.41) (end -53.46 53.21) (layer Edge.Cuts) (width 0.05))
 (gr_line (start -20.18158 62.523582) (end -35.44 55.41) (layer Edge.Cuts) (width 0.05))
 (gr_line (start -18.52 61.88) (end -12.39 48.741193) (layer Edge.Cuts) (width 0.05))
 (gr_arc (start -19.671581 61.373583) (end -20.18158 62.523582) (angle -90.17831882) (layer Edge.Cuts) (width 0.05))
 (gr_line (start -12.96244 47.07) (end -24.8 41.55) (layer Edge.Cuts) (width 0.05))
 (gr_arc (start -13.509999 48.191194) (end -12.39 48.741193) (angle -90.12474359) (layer Edge.Cuts) (width 0.05))
 (gr_arc (start -24.341167 40.382965) (end -25.561166 40.092966) (angle -81.90847125) (layer Edge.Cuts) (width 0.05))
 (gr_line (start -16.824085 -4.778756) (end -25.561166 40.092966) (layer Edge.Cuts) (width 0.05))
 (gr_arc (start -18.044084 -5.038755) (end -16.824085 -4.778756) (angle -90.27766385) (layer Edge.Cuts) (width 0.05))
 (gr_line (start -34.027391 -10.661237) (end -33.49 -13.43) (layer Edge.Cuts) (width 0.05))
 (gr_arc (start -32.797392 -10.451238) (end -34.027391 -10.661237) (angle -90.34411466) (layer Edge.Cuts) (width 0.05))
 (gr_line (start -17.79 -6.26) (end -33 -9.22) (layer Edge.Cuts) (width 0.05))
 (gr_line (start -94.79 -25.63) (end -79.227114 -25.63) (layer Edge.Cuts) (width 0.05))
 (gr_line (start -119.4 -2.62) (end -121.42 -14.058493) (layer Edge.Cuts) (width 0.05))
 (gr_line (start -140.321244 2.36) (end -120.389935 -1.14967) (layer Edge.Cuts) (width 0.05))
 (gr_arc (start -140.101245 3.589999) (end -140.321244 2.36) (angle -90.31911595) (layer Edge.Cuts) (width 0.05))
 (gr_arc (start -120.629934 -2.379669) (end -120.389935 -1.14967) (angle -90.0154728) (layer Edge.Cuts) (width 0.05))
 (gr_line (start -96.05 -20.83) (end -96.04 -24.38) (layer Edge.Cuts) (width 0.05))
 (gr_arc (start -97.303488 -20.83316) (end -97.142827 -19.590007) (angle -82.49165834) (layer Edge.Cuts) (width 0.05))
 (gr_line (start -120.370232 -15.49) (end -97.142827 -19.590007) (layer Edge.Cuts) (width 0.05))
 (gr_arc (start -120.180233 -14.250001) (end -120.370232 -15.49) (angle -90.06972518) (layer Edge.Cuts) (width 0.05))
 (gr_arc (start -76.74 -24.38) (end -77.99 -24.380066) (angle -81.73319074) (layer Edge.Cuts) (width 0.05))
 (gr_line (start -34.463874 -14.900785) (end -76.919794 -23.142998) (layer Edge.Cuts) (width 0.05))
 (gr_arc (start -34.709999 -13.679999) (end -33.49 -13.43) (angle -90.18185611) (layer Edge.Cuts) (width 0.05))
 (gr_arc (start -94.79 -24.38) (end -94.79 -25.63) (angle -90) (layer Edge.Cuts) (width 0.05))
 (gr_arc (start -79.24 -24.380066) (end -77.99 -24.380066) (angle -89.40934279) (layer Edge.Cuts) (width 0.05))
 (segment (start -61.97084 8.672188) (end -63.788115 9.897956) (width 0.25) (layer B.Cu) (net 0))
 (segment (start -65.332754 25.440768) (end -67.15003 26.666537) (width 0.25) (layer B.Cu) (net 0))
 (segment (start -59.150437 2.547824) (end -61.026336 3.813134) (width 0.25) (layer B.Cu) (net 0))
 (segment (start -62.512352 19.316405) (end -64.38825 20.581714) (width 0.25) (layer B.Cu) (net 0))
 (segment (start -64.38825 20.581714) (end -65.332754 25.440768) (width 0.25) (layer B.Cu) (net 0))
 (segment (start -61.026336 3.813134) (end -61.97084 8.672188) (width 0.25) (layer B.Cu) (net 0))
 (segment (start -104.481004 10.528075) (end -105.738301 12.323681) (width 0.25) (layer B.Cu) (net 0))
 (segment (start -101.627466 27.287171) (end -102.884763 29.082777) (width 0.25) (layer B.Cu) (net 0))
 (segment (start -104.042707 3.799746) (end -105.340563 5.653276) (width 0.25) (layer B.Cu) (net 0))
 (segment (start -108.690321 -4.418051) (end -107.351907 -6.329503) (width 0.25) (layer B.Cu) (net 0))
 (segment (start -108.788801 -4.400686) (end -108.690321 -4.418051) (width 0.25) (layer B.Cu) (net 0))
 (segment (start -101.189169 20.558843) (end -102.487025 22.412372) (width 0.25) (layer B.Cu) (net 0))
 (segment (start -102.487025 22.412372) (end -101.627466 27.287171) (width 0.25) (layer B.Cu) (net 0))
 (segment (start -105.340563 5.653276) (end -104.481004 10.528075) (width 0.25) (layer B.Cu) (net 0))
 (segment (start -106.91361 -13.057831) (end -108.211465 -11.204302) (width 0.25) (layer B.Cu) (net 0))
 (segment (start -108.211465 -11.204302) (end -107.351907 -6.329503) (width 0.25) (layer B.Cu) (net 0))
 (segment (start -117.866874 39.55448) (end -117.007318 44.429277) (width 0.25) (layer B.Cu) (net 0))
 (segment (start -119.664066 27.571402) (end -120.921365 29.367008) (width 0.25) (layer B.Cu) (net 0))
 (segment (start -117.007318 44.429277) (end -118.264613 46.224885) (width 0.25) (layer B.Cu) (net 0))
 (segment (start -119.225771 20.843076) (end -120.523627 22.696605) (width 0.25) (layer B.Cu) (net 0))
 (segment (start -128.606198 12.872967) (end -127.267786 10.961514) (width 0.25) (layer B.Cu) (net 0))
 (segment (start -128.70468 12.890331) (end -128.606198 12.872967) (width 0.25) (layer B.Cu) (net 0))
 (segment (start -116.569019 37.700951) (end -117.866874 39.55448) (width 0.25) (layer B.Cu) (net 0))
 (segment (start -120.523627 22.696605) (end -119.664066 27.571402) (width 0.25) (layer B.Cu) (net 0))
 (segment (start -128.127343 6.086715) (end -127.267786 10.961514) (width 0.25) (layer B.Cu) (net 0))
 (segment (start -126.829489 4.233186) (end -128.127343 6.086715) (width 0.25) (layer B.Cu) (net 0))
 (segment (start -17.366013 50.125313) (end -19.492295 50.899217) (width 0.25) (layer B.Cu) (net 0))
 (segment (start -23.867615 56.141267) (end -23.776982 56.183528) (width 0.25) (layer B.Cu) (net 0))
 (segment (start -19.492295 50.899217) (end -21.584255 55.385441) (width 0.25) (layer B.Cu) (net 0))
 (segment (start -23.776982 56.183528) (end -21.584255 55.385441) (width 0.25) (layer B.Cu) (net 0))
 (segment (start -61.133284 49.635676) (end -61.033664 49.626961) (width 0.25) (layer B.Cu) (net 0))
 (segment (start -39.664401 43.965422) (end -40.267653 48.878526) (width 0.25) (layer B.Cu) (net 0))
 (segment (start -42.106438 50.315143) (end -40.267653 48.878526) (width 0.25) (layer B.Cu) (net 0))
 (segment (start -42.205694 50.302955) (end -42.106438 50.315143) (width 0.25) (layer B.Cu) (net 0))
 (segment (start -40.876049 44.761173) (end -42.92679 45.717448) (width 0.25) (layer B.Cu) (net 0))
 (segment (start -55.87 -14.29) (end -57.745898 -13.024691) (width 0.25) (layer B.Cu) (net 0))
 (segment (start -57.635337 -13.053612) (end -58.579842 -8.194556) (width 0.25) (layer B.Cu) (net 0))
 (segment (start -60.514362 -6.889706) (end -58.579842 -8.194556) (width 0.25) (layer B.Cu) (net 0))
 (segment (start -60.612526 -6.908788) (end -60.514362 -6.889706) (width 0.25) (layer B.Cu) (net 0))
 (segment (start -81.916 -20.9) (end -83.516 -19.3) (width 0.25) (layer B.Cu) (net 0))
 (segment (start -83.516 -19.3) (end -83.516 -14.35) (width 0.25) (layer B.Cu) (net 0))
 (segment (start -85.266 -12.7) (end -85.166 -12.7) (width 0.25) (layer B.Cu) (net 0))
 (segment (start -85.166 -12.7) (end -83.516 -14.35) (width 0.25) (layer B.Cu) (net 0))
 (segment (start -82.016 -3.8) (end -83.616 -2.2) (width 0.25) (layer B.Cu) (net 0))
 (segment (start -83.616 -2.2) (end -83.616 2.75) (width 0.25) (layer B.Cu) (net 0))
 (segment (start -83.616 2.75) (end -85.166 4.3) (width 0.25) (layer B.Cu) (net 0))
 (segment (start -82.116 13.2) (end -83.716 14.8) (width 0.25) (layer B.Cu) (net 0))
 (segment (start -83.716 19.75) (end -85.266 21.3) (width 0.25) (layer B.Cu) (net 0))
 (segment (start -83.716 14.8) (end -83.716 19.75) (width 0.25) (layer B.Cu) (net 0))
 (segment (start -44.20084 12.122188) (end -46.018115 13.347956) (width 0.25) (layer B.Cu) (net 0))
 (segment (start -41.380437 5.997824) (end -43.256336 7.263134) (width 0.25) (layer B.Cu) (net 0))
 (segment (start -43.256336 7.263134) (end -44.20084 12.122188) (width 0.25) (layer B.Cu) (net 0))
 (segment (start -44.742352 22.766405) (end -46.61825 24.031714) (width 0.25) (layer B.Cu) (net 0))
 (segment (start -42.744362 -3.439706) (end -40.809842 -4.744556) (width 0.25) (layer B.Cu) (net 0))
 (segment (start -46.61825 24.031714) (end -47.562754 28.890768) (width 0.25) (layer B.Cu) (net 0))
 (segment (start -47.562754 28.890768) (end -49.38003 30.116537) (width 0.25) (layer B.Cu) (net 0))
 (segment (start -42.842526 -3.458788) (end -42.744362 -3.439706) (width 0.25) (layer B.Cu) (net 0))
 (segment (start -39.865337 -9.603612) (end -40.809842 -4.744556) (width 0.25) (layer B.Cu) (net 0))
 (segment (start -38.1 -10.84) (end -39.975898 -9.574691) (width 0.25) (layer B.Cu) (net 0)))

